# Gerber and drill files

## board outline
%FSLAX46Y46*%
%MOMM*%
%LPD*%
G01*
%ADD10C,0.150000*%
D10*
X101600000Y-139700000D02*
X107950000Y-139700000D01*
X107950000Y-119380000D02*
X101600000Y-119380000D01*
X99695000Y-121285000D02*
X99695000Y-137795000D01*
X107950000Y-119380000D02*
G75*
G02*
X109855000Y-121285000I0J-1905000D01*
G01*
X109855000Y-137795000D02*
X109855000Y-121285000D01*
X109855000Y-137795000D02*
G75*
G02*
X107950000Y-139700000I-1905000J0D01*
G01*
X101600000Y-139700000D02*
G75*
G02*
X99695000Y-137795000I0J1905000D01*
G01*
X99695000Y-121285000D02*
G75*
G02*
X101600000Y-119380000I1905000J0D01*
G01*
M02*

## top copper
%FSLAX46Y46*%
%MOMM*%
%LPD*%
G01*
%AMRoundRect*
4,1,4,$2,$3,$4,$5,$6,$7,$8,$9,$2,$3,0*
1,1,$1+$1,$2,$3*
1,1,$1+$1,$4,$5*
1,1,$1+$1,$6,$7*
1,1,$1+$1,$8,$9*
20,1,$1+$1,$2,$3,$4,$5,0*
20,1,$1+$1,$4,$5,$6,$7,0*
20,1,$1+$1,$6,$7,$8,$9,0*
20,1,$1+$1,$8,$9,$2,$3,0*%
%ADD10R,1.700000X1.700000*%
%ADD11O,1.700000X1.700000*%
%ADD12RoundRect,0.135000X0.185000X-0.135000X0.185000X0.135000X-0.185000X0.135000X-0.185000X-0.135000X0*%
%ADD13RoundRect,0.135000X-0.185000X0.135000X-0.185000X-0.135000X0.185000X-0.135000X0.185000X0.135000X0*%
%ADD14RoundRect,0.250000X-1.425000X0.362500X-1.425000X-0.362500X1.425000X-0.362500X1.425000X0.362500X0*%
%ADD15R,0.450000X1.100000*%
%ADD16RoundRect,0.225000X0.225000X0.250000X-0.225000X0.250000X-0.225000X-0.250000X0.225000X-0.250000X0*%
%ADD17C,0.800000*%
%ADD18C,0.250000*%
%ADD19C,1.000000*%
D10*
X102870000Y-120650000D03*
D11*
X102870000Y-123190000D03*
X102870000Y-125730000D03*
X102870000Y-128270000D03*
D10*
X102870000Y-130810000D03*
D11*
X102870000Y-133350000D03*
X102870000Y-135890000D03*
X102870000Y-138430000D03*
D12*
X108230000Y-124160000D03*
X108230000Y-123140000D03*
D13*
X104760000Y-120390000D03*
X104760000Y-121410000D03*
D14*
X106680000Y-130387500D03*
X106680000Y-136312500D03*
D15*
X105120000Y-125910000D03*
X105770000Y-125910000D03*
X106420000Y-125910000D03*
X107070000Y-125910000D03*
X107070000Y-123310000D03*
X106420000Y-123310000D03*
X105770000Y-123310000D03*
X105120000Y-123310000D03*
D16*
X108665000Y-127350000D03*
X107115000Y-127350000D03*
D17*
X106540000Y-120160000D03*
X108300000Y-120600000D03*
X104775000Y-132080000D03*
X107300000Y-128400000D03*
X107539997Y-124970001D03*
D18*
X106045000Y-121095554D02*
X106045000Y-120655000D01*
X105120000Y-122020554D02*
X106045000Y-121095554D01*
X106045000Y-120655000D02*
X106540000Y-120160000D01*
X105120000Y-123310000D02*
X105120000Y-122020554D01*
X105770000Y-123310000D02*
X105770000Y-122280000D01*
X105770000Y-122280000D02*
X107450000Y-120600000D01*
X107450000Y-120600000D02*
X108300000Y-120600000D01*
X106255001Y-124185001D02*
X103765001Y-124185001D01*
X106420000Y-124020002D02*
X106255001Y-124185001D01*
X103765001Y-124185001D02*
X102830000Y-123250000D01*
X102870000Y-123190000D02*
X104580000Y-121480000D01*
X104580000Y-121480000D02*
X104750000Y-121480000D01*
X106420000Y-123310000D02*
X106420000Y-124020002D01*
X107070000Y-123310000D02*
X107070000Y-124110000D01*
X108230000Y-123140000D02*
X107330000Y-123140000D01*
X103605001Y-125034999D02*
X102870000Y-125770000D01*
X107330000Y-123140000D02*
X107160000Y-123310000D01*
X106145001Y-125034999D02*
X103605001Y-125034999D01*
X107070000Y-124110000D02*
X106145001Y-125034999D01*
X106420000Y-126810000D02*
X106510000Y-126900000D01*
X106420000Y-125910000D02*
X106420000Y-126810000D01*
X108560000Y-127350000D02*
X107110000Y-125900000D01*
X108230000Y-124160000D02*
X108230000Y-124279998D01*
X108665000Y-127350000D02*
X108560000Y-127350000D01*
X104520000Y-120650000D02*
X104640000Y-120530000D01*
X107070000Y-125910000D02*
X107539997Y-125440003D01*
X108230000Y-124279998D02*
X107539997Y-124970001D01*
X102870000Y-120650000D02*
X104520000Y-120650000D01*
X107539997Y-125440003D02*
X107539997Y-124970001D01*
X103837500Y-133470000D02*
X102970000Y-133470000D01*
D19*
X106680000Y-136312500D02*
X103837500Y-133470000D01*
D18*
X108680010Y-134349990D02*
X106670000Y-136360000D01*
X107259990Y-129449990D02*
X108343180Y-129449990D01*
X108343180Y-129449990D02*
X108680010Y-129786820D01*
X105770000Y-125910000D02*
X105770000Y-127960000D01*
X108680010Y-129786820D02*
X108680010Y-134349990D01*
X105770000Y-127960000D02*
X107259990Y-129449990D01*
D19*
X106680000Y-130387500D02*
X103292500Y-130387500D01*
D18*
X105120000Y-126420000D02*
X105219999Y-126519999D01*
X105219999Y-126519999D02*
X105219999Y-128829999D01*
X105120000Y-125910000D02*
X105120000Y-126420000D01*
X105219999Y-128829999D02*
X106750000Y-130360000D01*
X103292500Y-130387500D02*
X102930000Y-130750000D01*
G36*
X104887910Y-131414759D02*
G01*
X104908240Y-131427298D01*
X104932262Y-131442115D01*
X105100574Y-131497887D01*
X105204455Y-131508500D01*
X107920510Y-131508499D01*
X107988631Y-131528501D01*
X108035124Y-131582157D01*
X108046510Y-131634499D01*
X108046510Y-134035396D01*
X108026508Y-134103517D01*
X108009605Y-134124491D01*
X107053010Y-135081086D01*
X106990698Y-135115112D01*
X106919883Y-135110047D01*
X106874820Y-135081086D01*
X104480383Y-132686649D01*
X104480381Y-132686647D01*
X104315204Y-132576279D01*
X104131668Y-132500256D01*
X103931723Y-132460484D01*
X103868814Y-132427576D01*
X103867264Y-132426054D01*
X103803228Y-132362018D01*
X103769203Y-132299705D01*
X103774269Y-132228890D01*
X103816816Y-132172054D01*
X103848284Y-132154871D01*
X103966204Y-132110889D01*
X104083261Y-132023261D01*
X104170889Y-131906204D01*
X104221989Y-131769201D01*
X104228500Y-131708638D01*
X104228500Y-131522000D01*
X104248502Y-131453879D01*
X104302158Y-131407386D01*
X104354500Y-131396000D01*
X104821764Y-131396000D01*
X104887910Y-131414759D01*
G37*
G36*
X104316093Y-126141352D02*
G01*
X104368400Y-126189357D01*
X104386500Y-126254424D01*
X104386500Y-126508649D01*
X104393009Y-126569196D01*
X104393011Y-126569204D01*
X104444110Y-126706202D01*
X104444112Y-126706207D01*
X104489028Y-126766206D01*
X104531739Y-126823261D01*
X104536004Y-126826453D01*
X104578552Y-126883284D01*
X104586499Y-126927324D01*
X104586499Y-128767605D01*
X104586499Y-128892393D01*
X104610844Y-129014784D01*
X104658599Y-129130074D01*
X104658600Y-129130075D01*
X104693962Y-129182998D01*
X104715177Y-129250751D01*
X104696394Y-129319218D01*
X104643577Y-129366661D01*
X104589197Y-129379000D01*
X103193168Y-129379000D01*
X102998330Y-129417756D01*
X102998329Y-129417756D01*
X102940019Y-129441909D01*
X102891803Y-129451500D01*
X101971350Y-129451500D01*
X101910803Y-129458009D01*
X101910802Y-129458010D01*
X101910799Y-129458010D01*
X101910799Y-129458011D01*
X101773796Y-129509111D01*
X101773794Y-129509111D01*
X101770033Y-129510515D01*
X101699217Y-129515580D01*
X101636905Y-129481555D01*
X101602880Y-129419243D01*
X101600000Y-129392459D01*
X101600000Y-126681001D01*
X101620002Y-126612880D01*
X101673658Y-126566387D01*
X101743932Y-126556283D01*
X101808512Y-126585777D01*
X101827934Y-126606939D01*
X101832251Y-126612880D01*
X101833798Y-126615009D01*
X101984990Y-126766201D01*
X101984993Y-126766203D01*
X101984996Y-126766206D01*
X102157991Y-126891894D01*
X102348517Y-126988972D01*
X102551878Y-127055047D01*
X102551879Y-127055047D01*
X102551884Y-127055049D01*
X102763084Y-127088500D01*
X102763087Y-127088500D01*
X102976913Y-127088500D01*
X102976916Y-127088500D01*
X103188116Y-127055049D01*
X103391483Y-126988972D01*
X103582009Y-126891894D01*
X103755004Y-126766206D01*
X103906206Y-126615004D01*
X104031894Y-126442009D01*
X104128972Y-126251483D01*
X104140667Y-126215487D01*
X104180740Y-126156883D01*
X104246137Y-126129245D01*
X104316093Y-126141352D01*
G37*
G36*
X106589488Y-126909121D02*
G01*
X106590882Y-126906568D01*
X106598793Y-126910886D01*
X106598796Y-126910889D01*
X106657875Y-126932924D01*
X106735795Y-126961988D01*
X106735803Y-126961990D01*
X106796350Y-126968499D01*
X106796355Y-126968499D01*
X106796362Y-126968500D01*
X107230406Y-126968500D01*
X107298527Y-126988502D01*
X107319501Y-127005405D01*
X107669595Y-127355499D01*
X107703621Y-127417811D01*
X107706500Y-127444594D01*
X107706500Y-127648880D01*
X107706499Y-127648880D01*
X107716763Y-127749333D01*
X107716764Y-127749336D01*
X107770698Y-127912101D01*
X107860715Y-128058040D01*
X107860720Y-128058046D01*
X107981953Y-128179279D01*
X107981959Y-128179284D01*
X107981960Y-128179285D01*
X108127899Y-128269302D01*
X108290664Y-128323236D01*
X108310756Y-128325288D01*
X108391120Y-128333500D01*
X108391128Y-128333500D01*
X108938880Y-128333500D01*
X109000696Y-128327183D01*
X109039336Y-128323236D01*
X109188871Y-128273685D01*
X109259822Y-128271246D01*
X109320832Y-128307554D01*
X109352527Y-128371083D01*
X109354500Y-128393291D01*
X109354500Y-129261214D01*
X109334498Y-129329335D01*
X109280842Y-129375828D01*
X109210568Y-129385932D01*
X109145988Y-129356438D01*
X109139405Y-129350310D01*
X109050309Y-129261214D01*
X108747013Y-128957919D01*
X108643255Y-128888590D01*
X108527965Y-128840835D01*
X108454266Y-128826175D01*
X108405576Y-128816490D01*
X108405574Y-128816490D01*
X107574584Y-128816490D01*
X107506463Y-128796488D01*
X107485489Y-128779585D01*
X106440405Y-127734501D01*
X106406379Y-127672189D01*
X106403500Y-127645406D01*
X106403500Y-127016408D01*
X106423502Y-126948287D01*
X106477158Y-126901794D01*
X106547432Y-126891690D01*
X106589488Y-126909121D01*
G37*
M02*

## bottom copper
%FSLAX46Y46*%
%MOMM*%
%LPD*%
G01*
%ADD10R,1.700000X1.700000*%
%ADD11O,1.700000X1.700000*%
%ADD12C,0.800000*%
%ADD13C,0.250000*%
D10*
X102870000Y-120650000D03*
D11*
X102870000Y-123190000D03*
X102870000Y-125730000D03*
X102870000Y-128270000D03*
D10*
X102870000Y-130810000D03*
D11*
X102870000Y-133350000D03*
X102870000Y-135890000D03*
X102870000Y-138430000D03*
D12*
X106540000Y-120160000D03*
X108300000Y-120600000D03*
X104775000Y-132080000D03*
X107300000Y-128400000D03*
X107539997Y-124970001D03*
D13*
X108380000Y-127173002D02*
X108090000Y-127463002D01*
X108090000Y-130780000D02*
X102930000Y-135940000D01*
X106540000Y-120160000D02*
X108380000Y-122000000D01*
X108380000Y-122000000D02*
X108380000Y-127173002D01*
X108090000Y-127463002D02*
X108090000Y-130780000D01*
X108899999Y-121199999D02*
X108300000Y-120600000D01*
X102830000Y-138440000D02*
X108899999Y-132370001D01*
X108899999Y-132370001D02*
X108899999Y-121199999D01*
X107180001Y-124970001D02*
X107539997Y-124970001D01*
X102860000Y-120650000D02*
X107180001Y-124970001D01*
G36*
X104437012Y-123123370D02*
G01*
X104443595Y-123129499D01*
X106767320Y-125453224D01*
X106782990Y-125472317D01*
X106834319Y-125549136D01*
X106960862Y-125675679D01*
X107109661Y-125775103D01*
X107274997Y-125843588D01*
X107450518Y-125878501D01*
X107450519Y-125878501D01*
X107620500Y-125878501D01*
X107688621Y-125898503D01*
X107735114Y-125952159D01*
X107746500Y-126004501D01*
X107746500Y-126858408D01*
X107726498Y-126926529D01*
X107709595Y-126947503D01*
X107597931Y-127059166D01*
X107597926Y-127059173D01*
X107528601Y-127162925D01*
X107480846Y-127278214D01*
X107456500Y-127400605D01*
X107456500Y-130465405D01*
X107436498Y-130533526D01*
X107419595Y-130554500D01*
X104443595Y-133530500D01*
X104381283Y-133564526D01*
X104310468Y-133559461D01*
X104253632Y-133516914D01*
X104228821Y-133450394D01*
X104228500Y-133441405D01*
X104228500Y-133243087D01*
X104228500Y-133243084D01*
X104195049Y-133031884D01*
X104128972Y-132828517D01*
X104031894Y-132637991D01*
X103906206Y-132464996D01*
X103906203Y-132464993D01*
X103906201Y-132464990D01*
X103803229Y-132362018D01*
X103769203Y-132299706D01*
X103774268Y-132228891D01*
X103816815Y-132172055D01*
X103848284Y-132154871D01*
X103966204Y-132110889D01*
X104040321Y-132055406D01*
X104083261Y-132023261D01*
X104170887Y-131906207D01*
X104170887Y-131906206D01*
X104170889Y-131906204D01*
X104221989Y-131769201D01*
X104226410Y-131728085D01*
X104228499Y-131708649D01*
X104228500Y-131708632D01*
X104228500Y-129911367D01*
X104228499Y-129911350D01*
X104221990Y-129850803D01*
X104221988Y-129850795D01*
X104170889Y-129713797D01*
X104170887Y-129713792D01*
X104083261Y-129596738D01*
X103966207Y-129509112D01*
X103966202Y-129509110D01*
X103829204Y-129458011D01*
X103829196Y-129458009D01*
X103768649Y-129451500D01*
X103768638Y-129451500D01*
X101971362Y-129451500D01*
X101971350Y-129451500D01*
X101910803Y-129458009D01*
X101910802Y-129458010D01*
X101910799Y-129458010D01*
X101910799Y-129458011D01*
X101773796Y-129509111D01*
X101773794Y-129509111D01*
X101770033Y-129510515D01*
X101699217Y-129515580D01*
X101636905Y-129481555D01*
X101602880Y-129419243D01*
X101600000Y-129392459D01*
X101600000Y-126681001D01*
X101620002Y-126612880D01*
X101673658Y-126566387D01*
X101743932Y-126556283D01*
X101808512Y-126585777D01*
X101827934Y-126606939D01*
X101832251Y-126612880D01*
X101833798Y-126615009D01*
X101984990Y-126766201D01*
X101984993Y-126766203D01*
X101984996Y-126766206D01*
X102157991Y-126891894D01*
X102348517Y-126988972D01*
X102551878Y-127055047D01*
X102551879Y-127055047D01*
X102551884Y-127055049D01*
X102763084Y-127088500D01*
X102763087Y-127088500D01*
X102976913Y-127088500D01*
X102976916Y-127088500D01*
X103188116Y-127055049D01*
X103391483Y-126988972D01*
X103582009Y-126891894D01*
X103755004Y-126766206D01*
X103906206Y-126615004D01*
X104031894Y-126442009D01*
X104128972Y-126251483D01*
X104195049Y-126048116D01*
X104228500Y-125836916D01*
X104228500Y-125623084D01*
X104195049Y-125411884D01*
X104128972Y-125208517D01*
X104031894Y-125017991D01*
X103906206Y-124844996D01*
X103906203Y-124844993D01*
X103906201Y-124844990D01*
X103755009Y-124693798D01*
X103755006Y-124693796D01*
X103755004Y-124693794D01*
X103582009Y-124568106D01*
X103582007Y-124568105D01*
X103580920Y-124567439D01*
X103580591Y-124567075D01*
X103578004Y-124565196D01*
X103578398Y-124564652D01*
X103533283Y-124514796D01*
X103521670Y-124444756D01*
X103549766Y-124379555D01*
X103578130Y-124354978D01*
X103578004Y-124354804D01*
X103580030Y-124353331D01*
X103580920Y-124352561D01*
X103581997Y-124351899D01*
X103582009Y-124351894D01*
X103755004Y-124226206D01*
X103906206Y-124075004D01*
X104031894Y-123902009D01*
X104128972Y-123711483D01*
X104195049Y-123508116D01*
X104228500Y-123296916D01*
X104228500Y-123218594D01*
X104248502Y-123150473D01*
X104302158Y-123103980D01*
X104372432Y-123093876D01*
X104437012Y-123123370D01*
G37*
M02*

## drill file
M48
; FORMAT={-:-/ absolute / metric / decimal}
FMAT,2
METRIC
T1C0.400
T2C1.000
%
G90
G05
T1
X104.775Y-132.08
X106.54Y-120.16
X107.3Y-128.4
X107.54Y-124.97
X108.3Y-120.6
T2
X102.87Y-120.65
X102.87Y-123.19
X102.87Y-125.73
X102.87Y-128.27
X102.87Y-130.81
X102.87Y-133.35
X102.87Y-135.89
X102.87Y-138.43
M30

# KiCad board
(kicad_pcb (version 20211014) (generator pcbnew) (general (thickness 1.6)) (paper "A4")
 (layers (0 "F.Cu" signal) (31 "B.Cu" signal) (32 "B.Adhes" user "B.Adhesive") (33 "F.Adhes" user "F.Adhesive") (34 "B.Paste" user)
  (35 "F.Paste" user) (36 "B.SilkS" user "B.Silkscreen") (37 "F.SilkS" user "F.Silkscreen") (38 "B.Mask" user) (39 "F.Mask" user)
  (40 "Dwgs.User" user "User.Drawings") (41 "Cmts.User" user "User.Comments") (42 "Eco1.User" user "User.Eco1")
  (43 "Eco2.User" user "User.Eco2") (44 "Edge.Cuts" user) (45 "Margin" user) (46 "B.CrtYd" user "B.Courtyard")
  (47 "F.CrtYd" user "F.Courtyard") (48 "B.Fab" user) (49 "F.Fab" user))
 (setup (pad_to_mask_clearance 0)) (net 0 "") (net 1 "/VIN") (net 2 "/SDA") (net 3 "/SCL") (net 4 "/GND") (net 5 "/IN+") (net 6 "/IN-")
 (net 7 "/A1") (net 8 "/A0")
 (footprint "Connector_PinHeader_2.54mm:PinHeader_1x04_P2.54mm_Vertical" (layer "F.Cu") (at 102.87 120.65)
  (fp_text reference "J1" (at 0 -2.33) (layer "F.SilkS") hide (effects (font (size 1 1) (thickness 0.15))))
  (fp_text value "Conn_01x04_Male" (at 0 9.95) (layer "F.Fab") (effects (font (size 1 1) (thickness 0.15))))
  (pad "1" thru_hole rect locked (at 0 0) (size 1.7 1.7) (drill 1) (layers *.Cu *.Mask) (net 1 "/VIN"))
  (pad "2" thru_hole oval locked (at 0 2.54) (size 1.7 1.7) (drill 1) (layers *.Cu *.Mask) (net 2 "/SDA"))
  (pad "3" thru_hole oval locked (at 0 5.08) (size 1.7 1.7) (drill 1) (layers *.Cu *.Mask) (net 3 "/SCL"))
  (pad "4" thru_hole oval locked (at 0 7.62) (size 1.7 1.7) (drill 1) (layers *.Cu *.Mask) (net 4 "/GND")))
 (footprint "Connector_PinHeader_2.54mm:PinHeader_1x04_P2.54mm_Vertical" (layer "F.Cu") (at 102.87 130.81)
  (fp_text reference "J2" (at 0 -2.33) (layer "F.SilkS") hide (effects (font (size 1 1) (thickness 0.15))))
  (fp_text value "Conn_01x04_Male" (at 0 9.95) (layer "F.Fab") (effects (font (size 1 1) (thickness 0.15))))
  (pad "1" thru_hole rect locked (at 0 0) (size 1.7 1.7) (drill 1) (layers *.Cu *.Mask) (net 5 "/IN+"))
  (pad "2" thru_hole oval locked (at 0 2.54) (size 1.7 1.7) (drill 1) (layers *.Cu *.Mask) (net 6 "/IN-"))
  (pad "3" thru_hole oval locked (at 0 5.08) (size 1.7 1.7) (drill 1) (layers *.Cu *.Mask) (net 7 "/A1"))
  (pad "4" thru_hole oval locked (at 0 7.62) (size 1.7 1.7) (drill 1) (layers *.Cu *.Mask) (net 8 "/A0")))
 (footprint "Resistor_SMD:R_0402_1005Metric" (layer "F.Cu") (at 108.23 123.65 90)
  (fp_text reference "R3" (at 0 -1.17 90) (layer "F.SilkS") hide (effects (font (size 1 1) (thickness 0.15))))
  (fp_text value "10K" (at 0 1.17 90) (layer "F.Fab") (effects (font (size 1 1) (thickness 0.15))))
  (pad "1" smd roundrect locked (at -0.51 0 90) (size 0.54 0.64) (layers "F.Cu" "F.Paste" "F.Mask") (roundrect_rratio 0.25) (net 1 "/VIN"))
  (pad "2" smd roundrect locked (at 0.51 0 90) (size 0.54 0.64) (layers "F.Cu" "F.Paste" "F.Mask") (roundrect_rratio 0.25) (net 3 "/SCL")))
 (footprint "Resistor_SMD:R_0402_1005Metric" (layer "F.Cu") (at 104.76 120.9 -90)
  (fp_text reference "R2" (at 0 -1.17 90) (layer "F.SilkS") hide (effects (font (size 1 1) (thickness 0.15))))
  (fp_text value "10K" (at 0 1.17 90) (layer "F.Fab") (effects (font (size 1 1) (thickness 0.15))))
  (pad "1" smd roundrect locked (at -0.51 0 270) (size 0.54 0.64) (layers "F.Cu" "F.Paste" "F.Mask") (roundrect_rratio 0.25) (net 1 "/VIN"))
  (pad "2" smd roundrect locked (at 0.51 0 270) (size 0.54 0.64) (layers "F.Cu" "F.Paste" "F.Mask") (roundrect_rratio 0.25) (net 2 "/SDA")))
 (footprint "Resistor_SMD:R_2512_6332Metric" (layer "F.Cu") (at 106.68 133.35 -90)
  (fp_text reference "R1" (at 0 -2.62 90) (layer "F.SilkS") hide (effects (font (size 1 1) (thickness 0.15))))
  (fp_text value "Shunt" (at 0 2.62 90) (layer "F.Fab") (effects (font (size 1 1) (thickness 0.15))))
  (pad "1" smd roundrect locked (at -2.9625 0 270) (size 1.225 3.35) (layers "F.Cu" "F.Paste" "F.Mask") (roundrect_rratio 0.2040816327)
   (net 5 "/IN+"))
  (pad "2" smd roundrect locked (at 2.9625 0 270) (size 1.225 3.35) (layers "F.Cu" "F.Paste" "F.Mask") (roundrect_rratio 0.2040816327)
   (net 6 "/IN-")))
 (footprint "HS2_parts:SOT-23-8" (layer "F.Cu") (at 105.12 125.91 90)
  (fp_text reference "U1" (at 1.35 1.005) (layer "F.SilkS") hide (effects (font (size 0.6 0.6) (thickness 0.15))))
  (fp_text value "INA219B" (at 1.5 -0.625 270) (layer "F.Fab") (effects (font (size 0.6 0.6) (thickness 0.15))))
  (pad "1" smd rect locked (at 0 0 90) (size 1.1 0.45) (layers "F.Cu" "F.Paste" "F.Mask") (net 5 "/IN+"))
  (pad "2" smd rect locked (at 0 0.65 90) (size 1.1 0.45) (layers "F.Cu" "F.Paste" "F.Mask") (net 6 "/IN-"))
  (pad "3" smd rect locked (at 0 1.3 90) (size 1.1 0.45) (layers "F.Cu" "F.Paste" "F.Mask") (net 4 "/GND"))
  (pad "4" smd rect locked (at 0 1.95 90) (size 1.1 0.45) (layers "F.Cu" "F.Paste" "F.Mask") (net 1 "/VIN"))
  (pad "5" smd rect locked (at 2.6 1.95 90) (size 1.1 0.45) (layers "F.Cu" "F.Paste" "F.Mask") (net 3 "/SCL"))
  (pad "6" smd rect locked (at 2.6 1.3 90) (size 1.1 0.45) (layers "F.Cu" "F.Paste" "F.Mask") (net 2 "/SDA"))
  (pad "7" smd rect locked (at 2.6 0.65 90) (size 1.1 0.45) (layers "F.Cu" "F.Paste" "F.Mask") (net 8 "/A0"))
  (pad "8" smd rect locked (at 2.6 0 90) (size 1.1 0.45) (layers "F.Cu" "F.Paste" "F.Mask") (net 7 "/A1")))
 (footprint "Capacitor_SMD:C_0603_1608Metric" (layer "F.Cu") (at 107.89 127.35 180)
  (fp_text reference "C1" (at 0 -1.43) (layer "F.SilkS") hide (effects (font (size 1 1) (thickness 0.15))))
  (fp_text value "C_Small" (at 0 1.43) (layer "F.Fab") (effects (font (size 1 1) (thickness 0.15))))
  (pad "1" smd roundrect locked (at -0.775 0 180) (size 0.9 0.95) (layers "F.Cu" "F.Paste" "F.Mask") (roundrect_rratio 0.25) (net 1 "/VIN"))
  (pad "2" smd roundrect locked (at 0.775 0 180) (size 0.9 0.95) (layers "F.Cu" "F.Paste" "F.Mask") (roundrect_rratio 0.25) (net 4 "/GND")))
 (gr_line (start 101.6 139.7) (end 107.95 139.7) (layer "Edge.Cuts") (width 0.15))
 (gr_line (start 107.95 119.38) (end 101.6 119.38) (layer "Edge.Cuts") (width 0.15))
 (gr_line (start 99.695 121.285) (end 99.695 137.795) (layer "Edge.Cuts") (width 0.15))
 (gr_arc (start 107.95 119.38) (mid 109.297038 119.937962) (end 109.855 121.285) (layer "Edge.Cuts") (width 0.15))
 (gr_line (start 109.855 137.795) (end 109.855 121.285) (layer "Edge.Cuts") (width 0.15))
 (gr_arc (start 109.855 137.795) (mid 109.297038 139.142038) (end 107.95 139.7) (layer "Edge.Cuts") (width 0.15))
 (gr_arc (start 101.6 139.7) (mid 100.252962 139.142038) (end 99.695 137.795) (layer "Edge.Cuts") (width 0.15))
 (gr_arc (start 99.695 121.285) (mid 100.252962 119.937962) (end 101.6 119.38) (layer "Edge.Cuts") (width 0.15))
 (segment (start 106.045 121.095554) (end 106.045 120.655) (width 0.25) (layer "F.Cu") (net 7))
 (segment (start 105.12 122.020554) (end 106.045 121.095554) (width 0.25) (layer "F.Cu") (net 7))
 (segment (start 106.045 120.655) (end 106.54 120.16) (width 0.25) (layer "F.Cu") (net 7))
 (segment (start 105.12 123.31) (end 105.12 122.020554) (width 0.25) (layer "F.Cu") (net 7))
 (via (at 106.54 120.16) (size 0.8) (drill 0.4) (layers "F.Cu" "B.Cu") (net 7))
 (segment (start 108.38 127.173002) (end 108.09 127.463002) (width 0.25) (layer "B.Cu") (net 7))
 (segment (start 108.09 130.78) (end 102.93 135.94) (width 0.25) (layer "B.Cu") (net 7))
 (segment (start 106.54 120.16) (end 108.38 122) (width 0.25) (layer "B.Cu") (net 7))
 (segment (start 108.38 122) (end 108.38 127.173002) (width 0.25) (layer "B.Cu") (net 7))
 (segment (start 108.09 127.463002) (end 108.09 130.78) (width 0.25) (layer "B.Cu") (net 7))
 (segment (start 105.77 123.31) (end 105.77 122.28) (width 0.25) (layer "F.Cu") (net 8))
 (segment (start 105.77 122.28) (end 107.45 120.6) (width 0.25) (layer "F.Cu") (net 8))
 (segment (start 107.45 120.6) (end 108.3 120.6) (width 0.25) (layer "F.Cu") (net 8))
 (via (at 108.3 120.6) (size 0.8) (drill 0.4) (layers "F.Cu" "B.Cu") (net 8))
 (segment (start 108.899999 121.199999) (end 108.3 120.6) (width 0.25) (layer "B.Cu") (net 8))
 (segment (start 102.83 138.44) (end 108.899999 132.370001) (width 0.25) (layer "B.Cu") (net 8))
 (segment (start 108.899999 132.370001) (end 108.899999 121.199999) (width 0.25) (layer "B.Cu") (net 8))
 (segment (start 106.255001 124.185001) (end 103.765001 124.185001) (width 0.25) (layer "F.Cu") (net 2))
 (segment (start 106.42 124.020002) (end 106.255001 124.185001) (width 0.25) (layer "F.Cu") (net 2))
 (segment (start 103.765001 124.185001) (end 102.83 123.25) (width 0.25) (layer "F.Cu") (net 2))
 (segment (start 102.87 123.19) (end 104.58 121.48) (width 0.25) (layer "F.Cu") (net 2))
 (segment (start 104.58 121.48) (end 104.75 121.48) (width 0.25) (layer "F.Cu") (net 2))
 (segment (start 106.42 123.31) (end 106.42 124.020002) (width 0.25) (layer "F.Cu") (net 2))
 (segment (start 107.07 123.31) (end 107.07 124.11) (width 0.25) (layer "F.Cu") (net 3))
 (segment (start 108.23 123.14) (end 107.33 123.14) (width 0.25) (layer "F.Cu") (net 3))
 (segment (start 103.605001 125.034999) (end 102.87 125.77) (width 0.25) (layer "F.Cu") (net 3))
 (segment (start 107.33 123.14) (end 107.16 123.31) (width 0.25) (layer "F.Cu") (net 3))
 (segment (start 106.145001 125.034999) (end 103.605001 125.034999) (width 0.25) (layer "F.Cu") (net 3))
 (segment (start 107.07 124.11) (end 106.145001 125.034999) (width 0.25) (layer "F.Cu") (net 3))
 (segment (start 106.42 126.81) (end 106.51 126.9) (width 0.25) (layer "F.Cu") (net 4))
 (segment (start 106.42 125.91) (end 106.42 126.81) (width 0.25) (layer "F.Cu") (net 4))
 (via (at 104.775 132.08) (size 0.8) (drill 0.4) (layers "F.Cu" "B.Cu") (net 4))
 (via (at 107.3 128.4) (size 0.8) (drill 0.4) (layers "F.Cu" "B.Cu") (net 4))
 (segment (start 108.56 127.35) (end 107.11 125.9) (width 0.25) (layer "F.Cu") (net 1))
 (segment (start 108.23 124.16) (end 108.23 124.279998) (width 0.25) (layer "F.Cu") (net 1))
 (segment (start 108.665 127.35) (end 108.56 127.35) (width 0.25) (layer "F.Cu") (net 1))
 (segment (start 104.52 120.65) (end 104.64 120.53) (width 0.25) (layer "F.Cu") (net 1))
 (segment (start 107.07 125.91) (end 107.539997 125.440003) (width 0.25) (layer "F.Cu") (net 1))
 (segment (start 108.23 124.279998) (end 107.539997 124.970001) (width 0.25) (layer "F.Cu") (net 1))
 (segment (start 102.87 120.65) (end 104.52 120.65) (width 0.25) (layer "F.Cu") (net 1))
 (segment (start 107.539997 125.440003) (end 107.539997 124.970001) (width 0.25) (layer "F.Cu") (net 1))
 (via (at 107.539997 124.970001) (size 0.8) (drill 0.4) (layers "F.Cu" "B.Cu") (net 1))
 (segment (start 107.180001 124.970001) (end 107.539997 124.970001) (width 0.25) (layer "B.Cu") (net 1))
 (segment (start 102.86 120.65) (end 107.180001 124.970001) (width 0.25) (layer "B.Cu") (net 1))
 (segment (start 103.8375 133.47) (end 102.97 133.47) (width 0.25) (layer "F.Cu") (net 6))
 (segment (start 106.68 136.3125) (end 103.8375 133.47) (width 1) (layer "F.Cu") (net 6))
 (segment (start 108.68001 134.34999) (end 106.67 136.36) (width 0.25) (layer "F.Cu") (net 6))
 (segment (start 107.25999 129.44999) (end 108.34318 129.44999) (width 0.25) (layer "F.Cu") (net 6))
 (segment (start 108.34318 129.44999) (end 108.68001 129.78682) (width 0.25) (layer "F.Cu") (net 6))
 (segment (start 105.77 125.91) (end 105.77 127.96) (width 0.25) (layer "F.Cu") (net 6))
 (segment (start 108.68001 129.78682) (end 108.68001 134.34999) (width 0.25) (layer "F.Cu") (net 6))
 (segment (start 105.77 127.96) (end 107.25999 129.44999) (width 0.25) (layer "F.Cu") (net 6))
 (segment (start 106.68 130.3875) (end 103.2925 130.3875) (width 1) (layer "F.Cu") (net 5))
 (segment (start 105.12 126.42) (end 105.219999 126.519999) (width 0.25) (layer "F.Cu") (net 5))
 (segment (start 105.219999 126.519999) (end 105.219999 128.829999) (width 0.25) (layer "F.Cu") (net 5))
 (segment (start 105.12 125.91) (end 105.12 126.42) (width 0.25) (layer "F.Cu") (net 5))
 (segment (start 105.219999 128.829999) (end 106.75 130.36) (width 0.25) (layer "F.Cu") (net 5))
 (segment (start 103.2925 130.3875) (end 102.93 130.75) (width 0.25) (layer "F.Cu") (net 5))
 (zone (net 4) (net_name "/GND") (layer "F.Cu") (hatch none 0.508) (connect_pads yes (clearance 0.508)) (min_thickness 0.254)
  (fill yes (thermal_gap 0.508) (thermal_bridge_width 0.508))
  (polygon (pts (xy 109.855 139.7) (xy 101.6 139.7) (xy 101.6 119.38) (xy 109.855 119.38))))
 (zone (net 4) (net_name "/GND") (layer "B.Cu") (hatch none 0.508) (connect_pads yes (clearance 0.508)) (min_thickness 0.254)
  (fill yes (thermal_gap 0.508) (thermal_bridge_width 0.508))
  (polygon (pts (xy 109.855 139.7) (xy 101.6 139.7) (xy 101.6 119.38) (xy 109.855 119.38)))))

